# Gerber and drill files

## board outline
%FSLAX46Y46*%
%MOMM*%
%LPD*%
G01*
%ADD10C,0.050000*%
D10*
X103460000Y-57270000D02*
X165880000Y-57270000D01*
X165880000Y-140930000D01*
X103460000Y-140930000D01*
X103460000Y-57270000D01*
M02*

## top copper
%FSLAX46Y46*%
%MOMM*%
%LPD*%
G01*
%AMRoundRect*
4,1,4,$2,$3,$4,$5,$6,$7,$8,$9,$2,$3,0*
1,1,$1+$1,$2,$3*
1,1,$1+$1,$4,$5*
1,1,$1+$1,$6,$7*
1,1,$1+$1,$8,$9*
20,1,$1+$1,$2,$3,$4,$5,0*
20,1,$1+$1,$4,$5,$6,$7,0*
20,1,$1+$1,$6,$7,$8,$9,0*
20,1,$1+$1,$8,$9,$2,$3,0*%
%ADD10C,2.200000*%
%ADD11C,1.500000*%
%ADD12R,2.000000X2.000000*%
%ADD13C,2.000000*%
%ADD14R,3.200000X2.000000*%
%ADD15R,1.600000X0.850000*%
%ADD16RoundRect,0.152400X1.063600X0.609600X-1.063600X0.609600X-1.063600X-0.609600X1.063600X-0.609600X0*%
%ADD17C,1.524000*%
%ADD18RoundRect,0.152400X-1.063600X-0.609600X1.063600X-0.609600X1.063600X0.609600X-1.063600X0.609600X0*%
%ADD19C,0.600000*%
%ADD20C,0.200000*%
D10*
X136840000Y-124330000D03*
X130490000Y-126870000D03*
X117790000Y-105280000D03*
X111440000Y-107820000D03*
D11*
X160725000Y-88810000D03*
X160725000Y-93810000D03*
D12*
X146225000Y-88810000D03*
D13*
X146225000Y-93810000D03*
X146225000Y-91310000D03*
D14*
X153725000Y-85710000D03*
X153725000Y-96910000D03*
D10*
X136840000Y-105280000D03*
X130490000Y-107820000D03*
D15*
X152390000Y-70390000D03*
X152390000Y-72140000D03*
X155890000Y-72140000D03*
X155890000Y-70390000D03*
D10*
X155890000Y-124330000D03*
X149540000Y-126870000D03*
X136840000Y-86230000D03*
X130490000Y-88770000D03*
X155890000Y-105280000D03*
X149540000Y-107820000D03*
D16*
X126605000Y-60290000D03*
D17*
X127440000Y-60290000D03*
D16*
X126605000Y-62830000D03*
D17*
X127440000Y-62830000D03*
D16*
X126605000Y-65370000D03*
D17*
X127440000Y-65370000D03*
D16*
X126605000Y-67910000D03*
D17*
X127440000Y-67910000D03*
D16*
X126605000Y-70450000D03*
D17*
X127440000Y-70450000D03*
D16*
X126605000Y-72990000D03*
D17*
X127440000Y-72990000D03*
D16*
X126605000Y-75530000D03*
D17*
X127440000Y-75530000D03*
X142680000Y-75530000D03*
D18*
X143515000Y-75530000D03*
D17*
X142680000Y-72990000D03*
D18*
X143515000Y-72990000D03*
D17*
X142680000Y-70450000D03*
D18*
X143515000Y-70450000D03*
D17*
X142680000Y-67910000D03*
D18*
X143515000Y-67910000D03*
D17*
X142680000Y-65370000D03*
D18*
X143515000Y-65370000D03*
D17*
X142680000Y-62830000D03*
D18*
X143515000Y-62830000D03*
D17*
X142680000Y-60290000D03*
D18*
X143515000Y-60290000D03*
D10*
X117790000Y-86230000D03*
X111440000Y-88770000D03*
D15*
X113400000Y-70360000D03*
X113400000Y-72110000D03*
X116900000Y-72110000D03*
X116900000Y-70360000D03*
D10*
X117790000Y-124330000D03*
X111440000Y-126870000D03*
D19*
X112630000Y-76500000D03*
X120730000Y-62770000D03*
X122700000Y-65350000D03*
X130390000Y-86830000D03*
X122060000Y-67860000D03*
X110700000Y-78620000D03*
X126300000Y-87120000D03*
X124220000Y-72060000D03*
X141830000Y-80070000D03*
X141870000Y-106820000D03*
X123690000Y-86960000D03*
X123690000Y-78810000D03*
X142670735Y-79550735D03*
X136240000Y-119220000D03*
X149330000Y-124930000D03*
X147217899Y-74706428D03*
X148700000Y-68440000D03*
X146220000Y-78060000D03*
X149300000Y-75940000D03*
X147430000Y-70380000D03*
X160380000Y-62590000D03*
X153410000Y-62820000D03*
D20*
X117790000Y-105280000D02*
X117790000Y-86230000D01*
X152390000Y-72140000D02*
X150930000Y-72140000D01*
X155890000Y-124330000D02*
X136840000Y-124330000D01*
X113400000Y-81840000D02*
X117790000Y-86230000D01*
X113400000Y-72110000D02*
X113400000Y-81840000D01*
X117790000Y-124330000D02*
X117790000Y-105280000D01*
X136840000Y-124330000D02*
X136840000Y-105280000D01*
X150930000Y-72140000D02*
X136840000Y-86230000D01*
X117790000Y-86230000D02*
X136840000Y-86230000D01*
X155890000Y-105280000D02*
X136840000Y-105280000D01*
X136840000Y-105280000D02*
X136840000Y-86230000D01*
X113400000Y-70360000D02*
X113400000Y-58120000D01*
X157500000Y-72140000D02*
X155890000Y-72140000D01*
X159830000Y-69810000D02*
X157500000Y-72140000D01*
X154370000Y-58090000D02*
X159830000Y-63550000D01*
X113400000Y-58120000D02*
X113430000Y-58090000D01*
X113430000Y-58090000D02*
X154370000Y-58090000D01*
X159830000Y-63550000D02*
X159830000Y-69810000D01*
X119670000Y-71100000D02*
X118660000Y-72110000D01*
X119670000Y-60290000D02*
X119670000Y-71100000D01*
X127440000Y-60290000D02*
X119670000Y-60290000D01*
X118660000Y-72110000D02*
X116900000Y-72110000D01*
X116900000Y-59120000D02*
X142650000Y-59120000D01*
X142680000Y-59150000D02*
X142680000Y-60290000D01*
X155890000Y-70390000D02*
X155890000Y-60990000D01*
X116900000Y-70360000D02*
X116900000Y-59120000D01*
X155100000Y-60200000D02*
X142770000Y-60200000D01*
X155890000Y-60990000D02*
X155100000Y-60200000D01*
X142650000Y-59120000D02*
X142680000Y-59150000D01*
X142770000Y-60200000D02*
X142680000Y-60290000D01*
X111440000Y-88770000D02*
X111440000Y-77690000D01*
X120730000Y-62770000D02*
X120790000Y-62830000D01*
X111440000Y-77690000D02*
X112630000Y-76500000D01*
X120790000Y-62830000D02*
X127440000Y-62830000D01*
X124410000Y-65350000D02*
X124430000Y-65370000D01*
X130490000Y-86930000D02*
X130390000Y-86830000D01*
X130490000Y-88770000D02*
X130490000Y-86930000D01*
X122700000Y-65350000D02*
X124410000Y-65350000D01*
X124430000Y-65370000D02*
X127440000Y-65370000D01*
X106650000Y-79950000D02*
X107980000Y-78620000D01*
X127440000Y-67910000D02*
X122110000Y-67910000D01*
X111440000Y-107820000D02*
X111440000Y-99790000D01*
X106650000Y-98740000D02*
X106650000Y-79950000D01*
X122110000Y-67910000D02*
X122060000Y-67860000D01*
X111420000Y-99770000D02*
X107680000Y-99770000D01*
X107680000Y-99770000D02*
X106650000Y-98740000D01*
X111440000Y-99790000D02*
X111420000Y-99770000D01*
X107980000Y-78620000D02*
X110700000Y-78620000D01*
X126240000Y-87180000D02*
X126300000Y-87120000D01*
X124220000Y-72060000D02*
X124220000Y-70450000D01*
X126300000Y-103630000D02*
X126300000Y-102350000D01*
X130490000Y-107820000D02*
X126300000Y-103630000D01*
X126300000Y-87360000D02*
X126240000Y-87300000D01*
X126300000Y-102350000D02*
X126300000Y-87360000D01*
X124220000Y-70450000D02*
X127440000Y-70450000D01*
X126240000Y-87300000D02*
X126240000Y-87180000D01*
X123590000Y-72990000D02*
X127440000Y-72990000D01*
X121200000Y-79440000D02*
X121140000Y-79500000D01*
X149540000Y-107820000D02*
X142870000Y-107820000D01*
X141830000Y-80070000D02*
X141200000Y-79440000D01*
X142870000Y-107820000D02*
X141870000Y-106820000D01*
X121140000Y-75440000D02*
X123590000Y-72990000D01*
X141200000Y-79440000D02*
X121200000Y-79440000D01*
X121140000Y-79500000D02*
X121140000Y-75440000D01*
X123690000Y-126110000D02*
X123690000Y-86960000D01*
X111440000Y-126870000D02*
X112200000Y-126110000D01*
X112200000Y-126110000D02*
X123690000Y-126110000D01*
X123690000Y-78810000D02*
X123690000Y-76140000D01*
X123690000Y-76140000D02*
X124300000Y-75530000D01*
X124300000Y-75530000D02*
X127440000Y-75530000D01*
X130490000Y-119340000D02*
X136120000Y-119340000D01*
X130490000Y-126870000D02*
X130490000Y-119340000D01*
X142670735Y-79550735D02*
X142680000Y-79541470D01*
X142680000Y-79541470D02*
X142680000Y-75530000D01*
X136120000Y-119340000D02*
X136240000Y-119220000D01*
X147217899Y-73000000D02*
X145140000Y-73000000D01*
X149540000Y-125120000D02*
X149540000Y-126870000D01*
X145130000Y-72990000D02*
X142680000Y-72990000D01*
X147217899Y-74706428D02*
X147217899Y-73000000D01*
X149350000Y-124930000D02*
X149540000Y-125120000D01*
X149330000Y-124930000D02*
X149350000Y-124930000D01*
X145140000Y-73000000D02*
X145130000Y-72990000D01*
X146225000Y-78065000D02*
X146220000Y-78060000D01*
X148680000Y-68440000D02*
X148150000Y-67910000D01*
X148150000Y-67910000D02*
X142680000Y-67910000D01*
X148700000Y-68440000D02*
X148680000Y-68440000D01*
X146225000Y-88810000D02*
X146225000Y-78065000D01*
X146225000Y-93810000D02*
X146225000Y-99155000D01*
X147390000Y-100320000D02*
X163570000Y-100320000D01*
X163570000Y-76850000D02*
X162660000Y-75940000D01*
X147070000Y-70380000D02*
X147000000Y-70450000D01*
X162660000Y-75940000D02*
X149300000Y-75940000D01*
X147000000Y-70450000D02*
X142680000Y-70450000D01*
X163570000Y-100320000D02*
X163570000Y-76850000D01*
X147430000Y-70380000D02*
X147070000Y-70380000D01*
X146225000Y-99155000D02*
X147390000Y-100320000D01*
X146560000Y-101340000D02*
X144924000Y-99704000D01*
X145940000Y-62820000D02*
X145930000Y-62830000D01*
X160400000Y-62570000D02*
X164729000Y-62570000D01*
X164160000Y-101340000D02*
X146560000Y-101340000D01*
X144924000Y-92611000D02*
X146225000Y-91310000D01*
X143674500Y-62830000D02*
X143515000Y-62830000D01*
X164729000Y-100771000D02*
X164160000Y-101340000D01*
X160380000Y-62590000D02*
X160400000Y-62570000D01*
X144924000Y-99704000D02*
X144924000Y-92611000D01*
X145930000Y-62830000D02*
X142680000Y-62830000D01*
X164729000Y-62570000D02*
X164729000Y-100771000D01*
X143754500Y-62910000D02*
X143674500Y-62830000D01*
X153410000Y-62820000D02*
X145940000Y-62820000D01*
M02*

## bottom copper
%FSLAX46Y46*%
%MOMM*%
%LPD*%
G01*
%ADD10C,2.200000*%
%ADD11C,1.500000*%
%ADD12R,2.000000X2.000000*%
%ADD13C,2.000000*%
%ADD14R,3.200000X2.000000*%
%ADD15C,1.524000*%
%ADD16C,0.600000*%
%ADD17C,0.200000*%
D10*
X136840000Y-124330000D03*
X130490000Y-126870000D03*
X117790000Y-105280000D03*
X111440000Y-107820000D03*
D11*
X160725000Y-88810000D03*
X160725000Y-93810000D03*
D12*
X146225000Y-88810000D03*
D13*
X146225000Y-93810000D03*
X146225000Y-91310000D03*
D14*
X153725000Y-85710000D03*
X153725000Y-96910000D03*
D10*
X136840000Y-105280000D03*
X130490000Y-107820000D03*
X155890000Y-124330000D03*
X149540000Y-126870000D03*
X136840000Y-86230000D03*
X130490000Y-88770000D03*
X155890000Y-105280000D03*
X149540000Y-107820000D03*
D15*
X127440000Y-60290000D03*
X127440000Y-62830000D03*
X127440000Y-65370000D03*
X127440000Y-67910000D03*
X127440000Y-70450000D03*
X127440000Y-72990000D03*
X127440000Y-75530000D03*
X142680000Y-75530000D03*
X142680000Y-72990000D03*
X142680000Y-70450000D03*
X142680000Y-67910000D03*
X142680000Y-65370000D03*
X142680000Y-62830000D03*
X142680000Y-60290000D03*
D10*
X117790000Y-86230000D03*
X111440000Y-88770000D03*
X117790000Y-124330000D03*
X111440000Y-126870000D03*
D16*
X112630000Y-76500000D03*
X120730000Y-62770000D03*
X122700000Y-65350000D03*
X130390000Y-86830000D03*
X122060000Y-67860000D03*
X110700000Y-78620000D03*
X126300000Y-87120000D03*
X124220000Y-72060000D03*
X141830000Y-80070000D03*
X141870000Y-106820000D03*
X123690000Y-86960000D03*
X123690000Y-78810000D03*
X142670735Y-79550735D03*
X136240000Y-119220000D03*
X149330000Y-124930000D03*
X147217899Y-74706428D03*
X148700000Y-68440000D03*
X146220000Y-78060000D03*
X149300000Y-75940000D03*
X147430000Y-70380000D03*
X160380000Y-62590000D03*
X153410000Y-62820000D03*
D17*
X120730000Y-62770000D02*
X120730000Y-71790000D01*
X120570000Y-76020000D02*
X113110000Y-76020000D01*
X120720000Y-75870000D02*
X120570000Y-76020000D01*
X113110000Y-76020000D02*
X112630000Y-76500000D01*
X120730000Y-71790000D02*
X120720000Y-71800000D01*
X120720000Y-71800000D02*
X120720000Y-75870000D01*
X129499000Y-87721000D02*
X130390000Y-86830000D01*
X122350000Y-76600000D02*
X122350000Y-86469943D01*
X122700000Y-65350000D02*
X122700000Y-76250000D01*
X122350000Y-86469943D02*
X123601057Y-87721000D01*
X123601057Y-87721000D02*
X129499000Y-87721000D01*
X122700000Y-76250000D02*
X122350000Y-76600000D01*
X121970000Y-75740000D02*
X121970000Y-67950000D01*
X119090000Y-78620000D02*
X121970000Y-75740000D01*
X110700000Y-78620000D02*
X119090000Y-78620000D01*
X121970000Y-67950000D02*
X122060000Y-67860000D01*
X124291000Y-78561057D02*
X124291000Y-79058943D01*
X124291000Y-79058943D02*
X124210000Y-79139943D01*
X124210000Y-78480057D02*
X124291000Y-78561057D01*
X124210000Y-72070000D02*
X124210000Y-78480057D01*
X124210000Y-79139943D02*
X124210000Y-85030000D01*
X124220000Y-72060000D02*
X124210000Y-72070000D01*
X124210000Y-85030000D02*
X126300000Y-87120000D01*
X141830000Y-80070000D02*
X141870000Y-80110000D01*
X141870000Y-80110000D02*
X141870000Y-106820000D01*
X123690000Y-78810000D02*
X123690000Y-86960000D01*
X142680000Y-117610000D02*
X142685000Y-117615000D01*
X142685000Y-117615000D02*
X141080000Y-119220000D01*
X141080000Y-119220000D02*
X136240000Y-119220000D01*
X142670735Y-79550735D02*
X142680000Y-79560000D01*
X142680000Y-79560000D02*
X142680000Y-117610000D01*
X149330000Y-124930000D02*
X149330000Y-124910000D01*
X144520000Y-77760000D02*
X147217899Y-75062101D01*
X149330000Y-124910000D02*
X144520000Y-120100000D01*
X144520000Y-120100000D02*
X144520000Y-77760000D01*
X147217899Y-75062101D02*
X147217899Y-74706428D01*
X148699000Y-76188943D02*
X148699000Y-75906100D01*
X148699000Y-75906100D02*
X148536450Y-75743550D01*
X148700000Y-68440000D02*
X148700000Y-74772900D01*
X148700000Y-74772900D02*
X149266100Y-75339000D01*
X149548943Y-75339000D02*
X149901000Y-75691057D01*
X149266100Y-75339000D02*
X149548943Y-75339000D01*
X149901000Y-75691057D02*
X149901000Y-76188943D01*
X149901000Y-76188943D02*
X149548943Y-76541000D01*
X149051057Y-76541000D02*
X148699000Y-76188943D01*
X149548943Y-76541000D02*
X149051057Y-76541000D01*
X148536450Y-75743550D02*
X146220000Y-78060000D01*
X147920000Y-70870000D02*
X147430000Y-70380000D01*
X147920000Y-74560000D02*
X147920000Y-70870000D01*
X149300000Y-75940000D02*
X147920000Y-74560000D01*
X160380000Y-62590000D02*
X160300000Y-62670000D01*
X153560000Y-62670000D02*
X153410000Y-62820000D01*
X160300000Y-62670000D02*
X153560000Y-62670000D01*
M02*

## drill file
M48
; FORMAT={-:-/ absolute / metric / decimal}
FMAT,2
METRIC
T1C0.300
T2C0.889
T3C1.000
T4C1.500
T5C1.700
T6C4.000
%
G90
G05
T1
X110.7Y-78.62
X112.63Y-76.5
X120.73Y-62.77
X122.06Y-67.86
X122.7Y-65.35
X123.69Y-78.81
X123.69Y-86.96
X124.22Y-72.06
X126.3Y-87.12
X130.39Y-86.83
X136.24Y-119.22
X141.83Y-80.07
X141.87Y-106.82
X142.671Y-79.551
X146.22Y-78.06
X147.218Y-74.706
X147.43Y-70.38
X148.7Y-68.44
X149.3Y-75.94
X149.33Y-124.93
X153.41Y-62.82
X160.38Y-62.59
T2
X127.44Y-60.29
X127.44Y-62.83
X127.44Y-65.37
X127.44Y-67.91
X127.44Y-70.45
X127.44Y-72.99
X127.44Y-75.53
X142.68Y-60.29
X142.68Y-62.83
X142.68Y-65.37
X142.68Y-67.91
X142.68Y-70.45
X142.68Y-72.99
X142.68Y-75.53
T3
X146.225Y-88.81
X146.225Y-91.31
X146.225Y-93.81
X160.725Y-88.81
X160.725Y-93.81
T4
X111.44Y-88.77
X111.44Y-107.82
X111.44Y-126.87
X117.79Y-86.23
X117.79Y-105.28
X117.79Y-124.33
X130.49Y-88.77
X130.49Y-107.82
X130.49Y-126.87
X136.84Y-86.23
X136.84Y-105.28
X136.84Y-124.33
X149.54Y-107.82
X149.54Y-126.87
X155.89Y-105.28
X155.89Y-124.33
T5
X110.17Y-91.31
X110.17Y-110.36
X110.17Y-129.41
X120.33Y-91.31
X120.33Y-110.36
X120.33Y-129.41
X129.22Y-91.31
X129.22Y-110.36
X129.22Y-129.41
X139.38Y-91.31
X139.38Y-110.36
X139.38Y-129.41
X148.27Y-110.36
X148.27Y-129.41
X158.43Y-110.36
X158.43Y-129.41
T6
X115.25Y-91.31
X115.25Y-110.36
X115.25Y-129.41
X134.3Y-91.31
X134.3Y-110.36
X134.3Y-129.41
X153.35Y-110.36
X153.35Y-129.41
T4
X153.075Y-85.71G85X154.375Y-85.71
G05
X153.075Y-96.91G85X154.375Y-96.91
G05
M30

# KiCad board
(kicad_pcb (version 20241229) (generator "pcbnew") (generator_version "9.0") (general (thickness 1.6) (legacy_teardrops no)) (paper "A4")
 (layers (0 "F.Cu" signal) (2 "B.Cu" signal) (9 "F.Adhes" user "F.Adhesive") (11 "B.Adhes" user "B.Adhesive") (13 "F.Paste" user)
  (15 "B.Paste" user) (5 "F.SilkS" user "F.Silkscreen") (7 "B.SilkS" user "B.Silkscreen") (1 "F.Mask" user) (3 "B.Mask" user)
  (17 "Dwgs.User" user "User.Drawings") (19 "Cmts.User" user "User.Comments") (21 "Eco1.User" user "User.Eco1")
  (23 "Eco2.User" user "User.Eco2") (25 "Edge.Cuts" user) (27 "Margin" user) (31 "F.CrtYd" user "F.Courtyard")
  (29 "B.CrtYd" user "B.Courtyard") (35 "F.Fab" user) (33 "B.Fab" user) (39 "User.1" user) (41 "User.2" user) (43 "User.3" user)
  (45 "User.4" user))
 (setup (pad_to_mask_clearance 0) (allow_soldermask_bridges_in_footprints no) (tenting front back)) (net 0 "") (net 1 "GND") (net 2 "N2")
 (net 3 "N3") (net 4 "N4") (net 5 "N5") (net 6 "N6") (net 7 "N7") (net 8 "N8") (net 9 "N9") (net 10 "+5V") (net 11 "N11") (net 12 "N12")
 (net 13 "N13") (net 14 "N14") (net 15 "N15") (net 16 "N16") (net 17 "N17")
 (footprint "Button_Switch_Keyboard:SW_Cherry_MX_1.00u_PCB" (layer "F.Cu") (at 136.84 124.33)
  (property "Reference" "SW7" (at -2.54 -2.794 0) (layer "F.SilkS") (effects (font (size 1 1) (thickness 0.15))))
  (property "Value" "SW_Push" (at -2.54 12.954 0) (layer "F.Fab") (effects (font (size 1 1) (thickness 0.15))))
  (pad "" np_thru_hole circle (at -7.62 5.08) (size 1.7 1.7) (drill 1.7) (layers "*.Cu" "*.Mask"))
  (pad "" np_thru_hole circle (at -2.54 5.08) (size 4 4) (drill 4) (layers "*.Cu" "*.Mask"))
  (pad "" np_thru_hole circle (at 2.54 5.08) (size 1.7 1.7) (drill 1.7) (layers "*.Cu" "*.Mask"))
  (pad "1" thru_hole circle (at 0 0) (size 2.2 2.2) (drill 1.5) (layers "*.Cu" "*.Mask") (remove_unused_layers no) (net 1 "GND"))
  (pad "2" thru_hole circle (at -6.35 2.54) (size 2.2 2.2) (drill 1.5) (layers "*.Cu" "*.Mask") (remove_unused_layers no) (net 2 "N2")))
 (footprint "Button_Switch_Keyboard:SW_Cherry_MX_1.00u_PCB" (layer "F.Cu") (at 117.79 105.28)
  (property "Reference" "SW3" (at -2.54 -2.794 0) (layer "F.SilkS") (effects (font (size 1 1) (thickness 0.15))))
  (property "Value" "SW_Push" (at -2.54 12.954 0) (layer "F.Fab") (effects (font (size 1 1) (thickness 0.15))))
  (pad "" np_thru_hole circle (at -7.62 5.08) (size 1.7 1.7) (drill 1.7) (layers "*.Cu" "*.Mask"))
  (pad "" np_thru_hole circle (at -2.54 5.08) (size 4 4) (drill 4) (layers "*.Cu" "*.Mask"))
  (pad "" np_thru_hole circle (at 2.54 5.08) (size 1.7 1.7) (drill 1.7) (layers "*.Cu" "*.Mask"))
  (pad "1" thru_hole circle (at 0 0) (size 2.2 2.2) (drill 1.5) (layers "*.Cu" "*.Mask") (remove_unused_layers no) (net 1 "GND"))
  (pad "2" thru_hole circle (at -6.35 2.54) (size 2.2 2.2) (drill 1.5) (layers "*.Cu" "*.Mask") (remove_unused_layers no) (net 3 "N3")))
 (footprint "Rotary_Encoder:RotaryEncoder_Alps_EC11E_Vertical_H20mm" (layer "F.Cu") (at 146.225 88.81)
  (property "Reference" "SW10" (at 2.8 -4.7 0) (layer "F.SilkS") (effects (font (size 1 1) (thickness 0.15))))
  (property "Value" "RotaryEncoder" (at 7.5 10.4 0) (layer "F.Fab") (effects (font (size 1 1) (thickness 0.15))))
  (pad "" thru_hole circle (at 14.5 0) (size 1.5 1.5) (drill 1) (layers "*.Cu" "*.Mask") (remove_unused_layers no))
  (pad "" thru_hole circle (at 14.5 5) (size 1.5 1.5) (drill 1) (layers "*.Cu" "*.Mask") (remove_unused_layers no))
  (pad "A" thru_hole rect (at 0 0) (size 2 2) (drill 1) (layers "*.Cu" "*.Mask") (remove_unused_layers no) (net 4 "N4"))
  (pad "B" thru_hole circle (at 0 5) (size 2 2) (drill 1) (layers "*.Cu" "*.Mask") (remove_unused_layers no) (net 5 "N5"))
  (pad "C" thru_hole circle (at 0 2.5) (size 2 2) (drill 1) (layers "*.Cu" "*.Mask") (remove_unused_layers no) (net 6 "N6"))
  (pad "MP" thru_hole rect (at 7.5 -3.1) (size 3.2 2) (drill oval 2.8 1.5) (layers "*.Cu" "*.Mask") (remove_unused_layers no))
  (pad "MP" thru_hole rect (at 7.5 8.1) (size 3.2 2) (drill oval 2.8 1.5) (layers "*.Cu" "*.Mask") (remove_unused_layers no)))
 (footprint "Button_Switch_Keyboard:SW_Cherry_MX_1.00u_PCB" (layer "F.Cu") (at 136.84 105.28)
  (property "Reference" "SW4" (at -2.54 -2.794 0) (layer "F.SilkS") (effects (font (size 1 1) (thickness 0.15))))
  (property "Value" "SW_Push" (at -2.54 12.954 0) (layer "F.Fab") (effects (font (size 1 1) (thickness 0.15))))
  (pad "" np_thru_hole circle (at -7.62 5.08) (size 1.7 1.7) (drill 1.7) (layers "*.Cu" "*.Mask"))
  (pad "" np_thru_hole circle (at -2.54 5.08) (size 4 4) (drill 4) (layers "*.Cu" "*.Mask"))
  (pad "" np_thru_hole circle (at 2.54 5.08) (size 1.7 1.7) (drill 1.7) (layers "*.Cu" "*.Mask"))
  (pad "1" thru_hole circle (at 0 0) (size 2.2 2.2) (drill 1.5) (layers "*.Cu" "*.Mask") (remove_unused_layers no) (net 1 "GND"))
  (pad "2" thru_hole circle (at -6.35 2.54) (size 2.2 2.2) (drill 1.5) (layers "*.Cu" "*.Mask") (remove_unused_layers no) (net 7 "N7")))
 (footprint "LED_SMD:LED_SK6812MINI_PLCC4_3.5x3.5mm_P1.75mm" (layer "F.Cu") (at 154.14 71.265)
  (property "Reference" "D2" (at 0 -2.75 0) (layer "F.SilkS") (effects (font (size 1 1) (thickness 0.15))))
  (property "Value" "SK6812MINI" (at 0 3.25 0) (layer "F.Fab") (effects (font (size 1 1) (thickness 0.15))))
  (pad "1" smd rect (at -1.75 -0.875) (size 1.6 0.85) (layers "F.Cu" "F.Mask" "F.Paste") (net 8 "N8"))
  (pad "2" smd rect (at -1.75 0.875) (size 1.6 0.85) (layers "F.Cu" "F.Mask" "F.Paste") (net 1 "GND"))
  (pad "3" smd rect (at 1.75 0.875) (size 1.6 0.85) (layers "F.Cu" "F.Mask" "F.Paste") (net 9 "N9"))
  (pad "4" smd rect (at 1.75 -0.875) (size 1.6 0.85) (layers "F.Cu" "F.Mask" "F.Paste") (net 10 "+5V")))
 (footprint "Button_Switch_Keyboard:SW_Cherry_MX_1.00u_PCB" (layer "F.Cu") (at 155.89 124.33)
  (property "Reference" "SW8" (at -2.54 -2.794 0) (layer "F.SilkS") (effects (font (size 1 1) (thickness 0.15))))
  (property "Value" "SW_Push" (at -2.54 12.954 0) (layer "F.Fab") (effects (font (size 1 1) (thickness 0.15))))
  (pad "" np_thru_hole circle (at -7.62 5.08) (size 1.7 1.7) (drill 1.7) (layers "*.Cu" "*.Mask"))
  (pad "" np_thru_hole circle (at -2.54 5.08) (size 4 4) (drill 4) (layers "*.Cu" "*.Mask"))
  (pad "" np_thru_hole circle (at 2.54 5.08) (size 1.7 1.7) (drill 1.7) (layers "*.Cu" "*.Mask"))
  (pad "1" thru_hole circle (at 0 0) (size 2.2 2.2) (drill 1.5) (layers "*.Cu" "*.Mask") (remove_unused_layers no) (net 1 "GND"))
  (pad "2" thru_hole circle (at -6.35 2.54) (size 2.2 2.2) (drill 1.5) (layers "*.Cu" "*.Mask") (remove_unused_layers no) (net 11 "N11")))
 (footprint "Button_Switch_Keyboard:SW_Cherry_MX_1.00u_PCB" (layer "F.Cu") (at 136.84 86.23)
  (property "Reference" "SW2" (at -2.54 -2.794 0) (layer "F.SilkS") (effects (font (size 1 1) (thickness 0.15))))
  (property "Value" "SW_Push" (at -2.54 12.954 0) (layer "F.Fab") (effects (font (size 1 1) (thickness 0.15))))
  (pad "" np_thru_hole circle (at -7.62 5.08) (size 1.7 1.7) (drill 1.7) (layers "*.Cu" "*.Mask"))
  (pad "" np_thru_hole circle (at -2.54 5.08) (size 4 4) (drill 4) (layers "*.Cu" "*.Mask"))
  (pad "" np_thru_hole circle (at 2.54 5.08) (size 1.7 1.7) (drill 1.7) (layers "*.Cu" "*.Mask"))
  (pad "1" thru_hole circle (at 0 0) (size 2.2 2.2) (drill 1.5) (layers "*.Cu" "*.Mask") (remove_unused_layers no) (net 1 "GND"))
  (pad "2" thru_hole circle (at -6.35 2.54) (size 2.2 2.2) (drill 1.5) (layers "*.Cu" "*.Mask") (remove_unused_layers no) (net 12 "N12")))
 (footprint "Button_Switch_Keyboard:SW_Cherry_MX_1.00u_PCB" (layer "F.Cu") (at 155.89 105.28)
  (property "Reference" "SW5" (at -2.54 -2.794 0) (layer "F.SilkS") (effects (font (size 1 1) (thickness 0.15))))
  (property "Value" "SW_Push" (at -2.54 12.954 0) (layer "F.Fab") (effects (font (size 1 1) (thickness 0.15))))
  (pad "" np_thru_hole circle (at -7.62 5.08) (size 1.7 1.7) (drill 1.7) (layers "*.Cu" "*.Mask"))
  (pad "" np_thru_hole circle (at -2.54 5.08) (size 4 4) (drill 4) (layers "*.Cu" "*.Mask"))
  (pad "" np_thru_hole circle (at 2.54 5.08) (size 1.7 1.7) (drill 1.7) (layers "*.Cu" "*.Mask"))
  (pad "1" thru_hole circle (at 0 0) (size 2.2 2.2) (drill 1.5) (layers "*.Cu" "*.Mask") (remove_unused_layers no) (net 1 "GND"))
  (pad "2" thru_hole circle (at -6.35 2.54) (size 2.2 2.2) (drill 1.5) (layers "*.Cu" "*.Mask") (remove_unused_layers no) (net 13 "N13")))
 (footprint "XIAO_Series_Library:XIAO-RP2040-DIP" (layer "F.Cu") (at 135.06 67.91)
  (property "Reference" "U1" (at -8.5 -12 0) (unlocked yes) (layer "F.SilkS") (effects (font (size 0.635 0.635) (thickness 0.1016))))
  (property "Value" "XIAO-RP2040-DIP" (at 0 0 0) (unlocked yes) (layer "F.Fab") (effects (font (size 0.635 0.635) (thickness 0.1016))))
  (pad "1" smd roundrect (at -8.455 -7.62 180) (size 2.432 1.524) (layers "F.Cu" "F.Mask") (roundrect_rratio 0.1) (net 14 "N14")
   (thermal_bridge_angle 45))
  (pad "1" thru_hole circle (at -7.62 -7.62 180) (size 1.524 1.524) (drill 0.889) (layers "*.Cu" "*.Mask") (remove_unused_layers no)
   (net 14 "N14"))
  (pad "2" smd roundrect (at -8.455 -5.08 180) (size 2.432 1.524) (layers "F.Cu" "F.Mask") (roundrect_rratio 0.1) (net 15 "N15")
   (thermal_bridge_angle 45))
  (pad "2" thru_hole circle (at -7.62 -5.08 180) (size 1.524 1.524) (drill 0.889) (layers "*.Cu" "*.Mask") (remove_unused_layers no)
   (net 15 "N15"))
  (pad "3" smd roundrect (at -8.455 -2.54 180) (size 2.432 1.524) (layers "F.Cu" "F.Mask") (roundrect_rratio 0.1) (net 12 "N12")
   (thermal_bridge_angle 45))
  (pad "3" thru_hole circle (at -7.62 -2.54 180) (size 1.524 1.524) (drill 0.889) (layers "*.Cu" "*.Mask") (remove_unused_layers no)
   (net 12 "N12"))
  (pad "4" smd roundrect (at -8.455 0 180) (size 2.432 1.524) (layers "F.Cu" "F.Mask") (roundrect_rratio 0.1) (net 3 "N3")
   (thermal_bridge_angle 45))
  (pad "4" thru_hole circle (at -7.62 0 180) (size 1.524 1.524) (drill 0.889) (layers "*.Cu" "*.Mask") (remove_unused_layers no)
   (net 3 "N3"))
  (pad "5" smd roundrect (at -8.455 2.54 180) (size 2.432 1.524) (layers "F.Cu" "F.Mask") (roundrect_rratio 0.1) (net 7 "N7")
   (thermal_bridge_angle 45))
  (pad "5" thru_hole circle (at -7.62 2.54 180) (size 1.524 1.524) (drill 0.889) (layers "*.Cu" "*.Mask") (remove_unused_layers no)
   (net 7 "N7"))
  (pad "6" smd roundrect (at -8.455 5.08 180) (size 2.432 1.524) (layers "F.Cu" "F.Mask") (roundrect_rratio 0.1) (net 13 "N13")
   (thermal_bridge_angle 45))
  (pad "6" thru_hole circle (at -7.62 5.08 180) (size 1.524 1.524) (drill 0.889) (layers "*.Cu" "*.Mask") (remove_unused_layers no)
   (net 13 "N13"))
  (pad "7" smd roundrect (at -8.455 7.62 180) (size 2.432 1.524) (layers "F.Cu" "F.Mask") (roundrect_rratio 0.1) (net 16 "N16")
   (thermal_bridge_angle 45))
  (pad "7" thru_hole circle (at -7.62 7.62 180) (size 1.524 1.524) (drill 0.889) (layers "*.Cu" "*.Mask") (remove_unused_layers no)
   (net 16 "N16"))
  (pad "8" thru_hole circle (at 7.62 7.62) (size 1.524 1.524) (drill 0.889) (layers "*.Cu" "*.Mask") (remove_unused_layers no) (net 2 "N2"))
  (pad "8" smd roundrect (at 8.455 7.62) (size 2.432 1.524) (layers "F.Cu" "F.Mask") (roundrect_rratio 0.1) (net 2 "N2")
   (thermal_bridge_angle 45))
  (pad "9" thru_hole circle (at 7.62 5.08) (size 1.524 1.524) (drill 0.889) (layers "*.Cu" "*.Mask") (remove_unused_layers no)
   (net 11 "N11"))
  (pad "9" smd roundrect (at 8.455 5.08) (size 2.432 1.524) (layers "F.Cu" "F.Mask") (roundrect_rratio 0.1) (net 11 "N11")
   (thermal_bridge_angle 45))
  (pad "10" thru_hole circle (at 7.62 2.54) (size 1.524 1.524) (drill 0.889) (layers "*.Cu" "*.Mask") (remove_unused_layers no) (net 5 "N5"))
  (pad "10" smd roundrect (at 8.455 2.54) (size 2.432 1.524) (layers "F.Cu" "F.Mask") (roundrect_rratio 0.1) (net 5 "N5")
   (thermal_bridge_angle 45))
  (pad "11" thru_hole circle (at 7.62 0) (size 1.524 1.524) (drill 0.889) (layers "*.Cu" "*.Mask") (remove_unused_layers no) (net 4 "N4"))
  (pad "11" smd roundrect (at 8.455 0) (size 2.432 1.524) (layers "F.Cu" "F.Mask") (roundrect_rratio 0.1) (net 4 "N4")
   (thermal_bridge_angle 45))
  (pad "12" thru_hole circle (at 7.62 -2.54) (size 1.524 1.524) (drill 0.889) (layers "*.Cu" "*.Mask") (remove_unused_layers no)
   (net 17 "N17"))
  (pad "12" smd roundrect (at 8.455 -2.54) (size 2.432 1.524) (layers "F.Cu" "F.Mask") (roundrect_rratio 0.1) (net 17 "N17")
   (thermal_bridge_angle 45))
  (pad "13" thru_hole circle (at 7.62 -5.08) (size 1.524 1.524) (drill 0.889) (layers "*.Cu" "*.Mask") (remove_unused_layers no)
   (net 6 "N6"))
  (pad "13" smd roundrect (at 8.455 -5.08) (size 2.432 1.524) (layers "F.Cu" "F.Mask") (roundrect_rratio 0.1) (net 6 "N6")
   (thermal_bridge_angle 45))
  (pad "14" thru_hole circle (at 7.62 -7.62) (size 1.524 1.524) (drill 0.889) (layers "*.Cu" "*.Mask") (remove_unused_layers no)
   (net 10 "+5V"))
  (pad "14" smd roundrect (at 8.455 -7.62) (size 2.432 1.524) (layers "F.Cu" "F.Mask") (roundrect_rratio 0.1) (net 10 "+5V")
   (thermal_bridge_angle 45)))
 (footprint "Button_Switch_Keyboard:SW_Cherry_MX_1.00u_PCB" (layer "F.Cu") (at 117.79 86.23)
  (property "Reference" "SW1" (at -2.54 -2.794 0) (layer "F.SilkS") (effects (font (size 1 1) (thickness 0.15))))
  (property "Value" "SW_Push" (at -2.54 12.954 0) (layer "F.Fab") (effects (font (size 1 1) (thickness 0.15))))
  (pad "" np_thru_hole circle (at -7.62 5.08) (size 1.7 1.7) (drill 1.7) (layers "*.Cu" "*.Mask"))
  (pad "" np_thru_hole circle (at -2.54 5.08) (size 4 4) (drill 4) (layers "*.Cu" "*.Mask"))
  (pad "" np_thru_hole circle (at 2.54 5.08) (size 1.7 1.7) (drill 1.7) (layers "*.Cu" "*.Mask"))
  (pad "1" thru_hole circle (at 0 0) (size 2.2 2.2) (drill 1.5) (layers "*.Cu" "*.Mask") (remove_unused_layers no) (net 1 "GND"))
  (pad "2" thru_hole circle (at -6.35 2.54) (size 2.2 2.2) (drill 1.5) (layers "*.Cu" "*.Mask") (remove_unused_layers no) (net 15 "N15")))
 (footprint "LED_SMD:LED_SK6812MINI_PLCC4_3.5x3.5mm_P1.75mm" (layer "F.Cu") (at 115.15 71.235)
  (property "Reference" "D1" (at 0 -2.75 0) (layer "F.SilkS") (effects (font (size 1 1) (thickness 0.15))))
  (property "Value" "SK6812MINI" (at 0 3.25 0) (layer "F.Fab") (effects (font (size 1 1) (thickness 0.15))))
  (pad "1" smd rect (at -1.75 -0.875) (size 1.6 0.85) (layers "F.Cu" "F.Mask" "F.Paste") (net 9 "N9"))
  (pad "2" smd rect (at -1.75 0.875) (size 1.6 0.85) (layers "F.Cu" "F.Mask" "F.Paste") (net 1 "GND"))
  (pad "3" smd rect (at 1.75 0.875) (size 1.6 0.85) (layers "F.Cu" "F.Mask" "F.Paste") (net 14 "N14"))
  (pad "4" smd rect (at 1.75 -0.875) (size 1.6 0.85) (layers "F.Cu" "F.Mask" "F.Paste") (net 10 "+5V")))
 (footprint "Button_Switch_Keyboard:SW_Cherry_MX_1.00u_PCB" (layer "F.Cu") (at 117.79 124.33)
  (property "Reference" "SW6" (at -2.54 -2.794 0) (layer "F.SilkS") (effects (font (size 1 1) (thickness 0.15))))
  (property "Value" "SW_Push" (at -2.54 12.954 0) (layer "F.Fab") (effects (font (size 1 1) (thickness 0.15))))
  (pad "" np_thru_hole circle (at -7.62 5.08) (size 1.7 1.7) (drill 1.7) (layers "*.Cu" "*.Mask"))
  (pad "" np_thru_hole circle (at -2.54 5.08) (size 4 4) (drill 4) (layers "*.Cu" "*.Mask"))
  (pad "" np_thru_hole circle (at 2.54 5.08) (size 1.7 1.7) (drill 1.7) (layers "*.Cu" "*.Mask"))
  (pad "1" thru_hole circle (at 0 0) (size 2.2 2.2) (drill 1.5) (layers "*.Cu" "*.Mask") (remove_unused_layers no) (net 1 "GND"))
  (pad "2" thru_hole circle (at -6.35 2.54) (size 2.2 2.2) (drill 1.5) (layers "*.Cu" "*.Mask") (remove_unused_layers no) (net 16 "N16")))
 (gr_rect (start 103.46 57.27) (end 165.88 140.93) (stroke (width 0.05) (type default)) (fill no) (layer "Edge.Cuts"))
 (segment (start 117.79 105.28) (end 117.79 86.23) (width 0.2) (layer "F.Cu") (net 1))
 (segment (start 152.39 72.14) (end 150.93 72.14) (width 0.2) (layer "F.Cu") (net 1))
 (segment (start 155.89 124.33) (end 136.84 124.33) (width 0.2) (layer "F.Cu") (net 1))
 (segment (start 113.4 81.84) (end 117.79 86.23) (width 0.2) (layer "F.Cu") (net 1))
 (segment (start 113.4 72.11) (end 113.4 81.84) (width 0.2) (layer "F.Cu") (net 1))
 (segment (start 117.79 124.33) (end 117.79 105.28) (width 0.2) (layer "F.Cu") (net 1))
 (segment (start 136.84 124.33) (end 136.84 105.28) (width 0.2) (layer "F.Cu") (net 1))
 (segment (start 150.93 72.14) (end 136.84 86.23) (width 0.2) (layer "F.Cu") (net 1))
 (segment (start 117.79 86.23) (end 136.84 86.23) (width 0.2) (layer "F.Cu") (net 1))
 (segment (start 155.89 105.28) (end 136.84 105.28) (width 0.2) (layer "F.Cu") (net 1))
 (segment (start 136.84 105.28) (end 136.84 86.23) (width 0.2) (layer "F.Cu") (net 1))
 (segment (start 113.4 70.36) (end 113.4 58.12) (width 0.2) (layer "F.Cu") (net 9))
 (segment (start 157.5 72.14) (end 155.89 72.14) (width 0.2) (layer "F.Cu") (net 9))
 (segment (start 159.83 69.81) (end 157.5 72.14) (width 0.2) (layer "F.Cu") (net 9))
 (segment (start 154.37 58.09) (end 159.83 63.55) (width 0.2) (layer "F.Cu") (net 9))
 (segment (start 113.4 58.12) (end 113.43 58.09) (width 0.2) (layer "F.Cu") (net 9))
 (segment (start 113.43 58.09) (end 154.37 58.09) (width 0.2) (layer "F.Cu") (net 9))
 (segment (start 159.83 63.55) (end 159.83 69.81) (width 0.2) (layer "F.Cu") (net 9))
 (segment (start 119.67 71.1) (end 118.66 72.11) (width 0.2) (layer "F.Cu") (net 14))
 (segment (start 119.67 60.29) (end 119.67 71.1) (width 0.2) (layer "F.Cu") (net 14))
 (segment (start 127.44 60.29) (end 119.67 60.29) (width 0.2) (layer "F.Cu") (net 14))
 (segment (start 118.66 72.11) (end 116.9 72.11) (width 0.2) (layer "F.Cu") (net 14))
 (segment (start 116.9 59.12) (end 142.65 59.12) (width 0.2) (layer "F.Cu") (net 10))
 (segment (start 142.68 59.15) (end 142.68 60.29) (width 0.2) (layer "F.Cu") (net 10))
 (segment (start 155.89 70.39) (end 155.89 60.99) (width 0.2) (layer "F.Cu") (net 10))
 (segment (start 116.9 70.36) (end 116.9 59.12) (width 0.2) (layer "F.Cu") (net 10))
 (segment (start 155.1 60.2) (end 142.77 60.2) (width 0.2) (layer "F.Cu") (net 10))
 (segment (start 155.89 60.99) (end 155.1 60.2) (width 0.2) (layer "F.Cu") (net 10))
 (segment (start 142.65 59.12) (end 142.68 59.15) (width 0.2) (layer "F.Cu") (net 10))
 (segment (start 142.77 60.2) (end 142.68 60.29) (width 0.2) (layer "F.Cu") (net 10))
 (segment (start 111.44 88.77) (end 111.44 77.69) (width 0.2) (layer "F.Cu") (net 15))
 (segment (start 120.73 62.77) (end 120.79 62.83) (width 0.2) (layer "F.Cu") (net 15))
 (segment (start 111.44 77.69) (end 112.63 76.5) (width 0.2) (layer "F.Cu") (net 15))
 (segment (start 120.79 62.83) (end 127.44 62.83) (width 0.2) (layer "F.Cu") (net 15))
 (via (at 112.63 76.5) (size 0.6) (drill 0.3) (layers "F.Cu" "B.Cu") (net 15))
 (via (at 120.73 62.77) (size 0.6) (drill 0.3) (layers "F.Cu" "B.Cu") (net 15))
 (segment (start 120.73 62.77) (end 120.73 71.79) (width 0.2) (layer "B.Cu") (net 15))
 (segment (start 120.57 76.02) (end 113.11 76.02) (width 0.2) (layer "B.Cu") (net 15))
 (segment (start 120.72 75.87) (end 120.57 76.02) (width 0.2) (layer "B.Cu") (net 15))
 (segment (start 113.11 76.02) (end 112.63 76.5) (width 0.2) (layer "B.Cu") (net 15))
 (segment (start 120.73 71.79) (end 120.72 71.8) (width 0.2) (layer "B.Cu") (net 15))
 (segment (start 120.72 71.8) (end 120.72 75.87) (width 0.2) (layer "B.Cu") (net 15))
 (segment (start 124.41 65.35) (end 124.43 65.37) (width 0.2) (layer "F.Cu") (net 12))
 (segment (start 130.49 86.93) (end 130.39 86.83) (width 0.2) (layer "F.Cu") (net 12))
 (segment (start 130.49 88.77) (end 130.49 86.93) (width 0.2) (layer "F.Cu") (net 12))
 (segment (start 122.7 65.35) (end 124.41 65.35) (width 0.2) (layer "F.Cu") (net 12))
 (segment (start 124.43 65.37) (end 127.44 65.37) (width 0.2) (layer "F.Cu") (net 12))
 (via (at 122.7 65.35) (size 0.6) (drill 0.3) (layers "F.Cu" "B.Cu") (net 12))
 (via (at 130.39 86.83) (size 0.6) (drill 0.3) (layers "F.Cu" "B.Cu") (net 12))
 (segment (start 129.499 87.721) (end 130.39 86.83) (width 0.2) (layer "B.Cu") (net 12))
 (segment (start 122.35 76.6) (end 122.35 86.469943) (width 0.2) (layer "B.Cu") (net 12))
 (segment (start 122.7 65.35) (end 122.7 76.25) (width 0.2) (layer "B.Cu") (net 12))
 (segment (start 122.35 86.469943) (end 123.601057 87.721) (width 0.2) (layer "B.Cu") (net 12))
 (segment (start 123.601057 87.721) (end 129.499 87.721) (width 0.2) (layer "B.Cu") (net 12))
 (segment (start 122.7 76.25) (end 122.35 76.6) (width 0.2) (layer "B.Cu") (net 12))
 (segment (start 106.65 79.95) (end 107.98 78.62) (width 0.2) (layer "F.Cu") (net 3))
 (segment (start 127.44 67.91) (end 122.11 67.91) (width 0.2) (layer "F.Cu") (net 3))
 (segment (start 111.44 107.82) (end 111.44 99.79) (width 0.2) (layer "F.Cu") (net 3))
 (segment (start 106.65 98.74) (end 106.65 79.95) (width 0.2) (layer "F.Cu") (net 3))
 (segment (start 122.11 67.91) (end 122.06 67.86) (width 0.2) (layer "F.Cu") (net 3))
 (segment (start 111.42 99.77) (end 107.68 99.77) (width 0.2) (layer "F.Cu") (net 3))
 (segment (start 107.68 99.77) (end 106.65 98.74) (width 0.2) (layer "F.Cu") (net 3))
 (segment (start 111.44 99.79) (end 111.42 99.77) (width 0.2) (layer "F.Cu") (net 3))
 (segment (start 107.98 78.62) (end 110.7 78.62) (width 0.2) (layer "F.Cu") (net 3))
 (via (at 122.06 67.86) (size 0.6) (drill 0.3) (layers "F.Cu" "B.Cu") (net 3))
 (via (at 110.7 78.62) (size 0.6) (drill 0.3) (layers "F.Cu" "B.Cu") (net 3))
 (segment (start 121.97 75.74) (end 121.97 67.95) (width 0.2) (layer "B.Cu") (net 3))
 (segment (start 119.09 78.62) (end 121.97 75.74) (width 0.2) (layer "B.Cu") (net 3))
 (segment (start 110.7 78.62) (end 119.09 78.62) (width 0.2) (layer "B.Cu") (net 3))
 (segment (start 121.97 67.95) (end 122.06 67.86) (width 0.2) (layer "B.Cu") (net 3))
 (segment (start 126.24 87.18) (end 126.3 87.12) (width 0.2) (layer "F.Cu") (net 7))
 (segment (start 124.22 72.06) (end 124.22 70.45) (width 0.2) (layer "F.Cu") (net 7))
 (segment (start 126.3 103.63) (end 126.3 102.35) (width 0.2) (layer "F.Cu") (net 7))
 (segment (start 130.49 107.82) (end 126.3 103.63) (width 0.2) (layer "F.Cu") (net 7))
 (segment (start 126.3 87.36) (end 126.24 87.3) (width 0.2) (layer "F.Cu") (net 7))
 (segment (start 126.3 102.35) (end 126.3 87.36) (width 0.2) (layer "F.Cu") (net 7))
 (segment (start 124.22 70.45) (end 127.44 70.45) (width 0.2) (layer "F.Cu") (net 7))
 (segment (start 126.24 87.3) (end 126.24 87.18) (width 0.2) (layer "F.Cu") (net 7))
 (via (at 126.3 87.12) (size 0.6) (drill 0.3) (layers "F.Cu" "B.Cu") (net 7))
 (via (at 124.22 72.06) (size 0.6) (drill 0.3) (layers "F.Cu" "B.Cu") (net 7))
 (segment (start 124.291 78.561057) (end 124.291 79.058943) (width 0.2) (layer "B.Cu") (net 7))
 (segment (start 124.291 79.058943) (end 124.21 79.139943) (width 0.2) (layer "B.Cu") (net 7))
 (segment (start 124.21 78.480057) (end 124.291 78.561057) (width 0.2) (layer "B.Cu") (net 7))
 (segment (start 124.21 72.07) (end 124.21 78.480057) (width 0.2) (layer "B.Cu") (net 7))
 (segment (start 124.21 79.139943) (end 124.21 85.03) (width 0.2) (layer "B.Cu") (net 7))
 (segment (start 124.22 72.06) (end 124.21 72.07) (width 0.2) (layer "B.Cu") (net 7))
 (segment (start 124.21 85.03) (end 126.3 87.12) (width 0.2) (layer "B.Cu") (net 7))
 (segment (start 123.59 72.99) (end 127.44 72.99) (width 0.2) (layer "F.Cu") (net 13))
 (segment (start 121.2 79.44) (end 121.14 79.5) (width 0.2) (layer "F.Cu") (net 13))
 (segment (start 149.54 107.82) (end 142.87 107.82) (width 0.2) (layer "F.Cu") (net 13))
 (segment (start 141.83 80.07) (end 141.2 79.44) (width 0.2) (layer "F.Cu") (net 13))
 (segment (start 142.87 107.82) (end 141.87 106.82) (width 0.2) (layer "F.Cu") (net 13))
 (segment (start 121.14 75.44) (end 123.59 72.99) (width 0.2) (layer "F.Cu") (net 13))
 (segment (start 141.2 79.44) (end 121.2 79.44) (width 0.2) (layer "F.Cu") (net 13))
 (segment (start 121.14 79.5) (end 121.14 75.44) (width 0.2) (layer "F.Cu") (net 13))
 (via (at 141.83 80.07) (size 0.6) (drill 0.3) (layers "F.Cu" "B.Cu") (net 13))
 (via (at 141.87 106.82) (size 0.6) (drill 0.3) (layers "F.Cu" "B.Cu") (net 13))
 (segment (start 141.83 80.07) (end 141.87 80.11) (width 0.2) (layer "B.Cu") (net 13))
 (segment (start 141.87 80.11) (end 141.87 106.82) (width 0.2) (layer "B.Cu") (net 13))
 (segment (start 123.69 126.11) (end 123.69 86.96) (width 0.2) (layer "F.Cu") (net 16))
 (segment (start 111.44 126.87) (end 112.2 126.11) (width 0.2) (layer "F.Cu") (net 16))
 (segment (start 112.2 126.11) (end 123.69 126.11) (width 0.2) (layer "F.Cu") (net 16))
 (segment (start 123.69 78.81) (end 123.69 76.14) (width 0.2) (layer "F.Cu") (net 16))
 (segment (start 123.69 76.14) (end 124.3 75.53) (width 0.2) (layer "F.Cu") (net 16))
 (segment (start 124.3 75.53) (end 127.44 75.53) (width 0.2) (layer "F.Cu") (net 16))
 (via (at 123.69 86.96) (size 0.6) (drill 0.3) (layers "F.Cu" "B.Cu") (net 16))
 (via (at 123.69 78.81) (size 0.6) (drill 0.3) (layers "F.Cu" "B.Cu") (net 16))
 (segment (start 123.69 78.81) (end 123.69 86.96) (width 0.2) (layer "B.Cu") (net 16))
 (segment (start 130.49 119.34) (end 136.12 119.34) (width 0.2) (layer "F.Cu") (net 2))
 (segment (start 130.49 126.87) (end 130.49 119.34) (width 0.2) (layer "F.Cu") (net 2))
 (segment (start 142.670735 79.550735) (end 142.68 79.54147) (width 0.2) (layer "F.Cu") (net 2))
 (segment (start 142.68 79.54147) (end 142.68 75.53) (width 0.2) (layer "F.Cu") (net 2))
 (segment (start 136.12 119.34) (end 136.24 119.22) (width 0.2) (layer "F.Cu") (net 2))
 (via (at 142.670735 79.550735) (size 0.6) (drill 0.3) (layers "F.Cu" "B.Cu") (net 2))
 (via (at 136.24 119.22) (size 0.6) (drill 0.3) (layers "F.Cu" "B.Cu") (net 2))
 (segment (start 142.68 117.61) (end 142.685 117.615) (width 0.2) (layer "B.Cu") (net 2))
 (segment (start 142.685 117.615) (end 141.08 119.22) (width 0.2) (layer "B.Cu") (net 2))
 (segment (start 141.08 119.22) (end 136.24 119.22) (width 0.2) (layer "B.Cu") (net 2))
 (segment (start 142.670735 79.550735) (end 142.68 79.56) (width 0.2) (layer "B.Cu") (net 2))
 (segment (start 142.68 79.56) (end 142.68 117.61) (width 0.2) (layer "B.Cu") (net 2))
 (segment (start 147.217899 73) (end 145.14 73) (width 0.2) (layer "F.Cu") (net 11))
 (segment (start 149.54 125.12) (end 149.54 126.87) (width 0.2) (layer "F.Cu") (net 11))
 (segment (start 145.13 72.99) (end 142.68 72.99) (width 0.2) (layer "F.Cu") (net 11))
 (segment (start 147.217899 74.706428) (end 147.217899 73) (width 0.2) (layer "F.Cu") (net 11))
 (segment (start 149.35 124.93) (end 149.54 125.12) (width 0.2) (layer "F.Cu") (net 11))
 (segment (start 149.33 124.93) (end 149.35 124.93) (width 0.2) (layer "F.Cu") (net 11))
 (segment (start 145.14 73) (end 145.13 72.99) (width 0.2) (layer "F.Cu") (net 11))
 (via (at 149.33 124.93) (size 0.6) (drill 0.3) (layers "F.Cu" "B.Cu") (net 11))
 (via (at 147.217899 74.706428) (size 0.6) (drill 0.3) (layers "F.Cu" "B.Cu") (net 11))
 (segment (start 149.33 124.93) (end 149.33 124.91) (width 0.2) (layer "B.Cu") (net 11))
 (segment (start 144.52 77.76) (end 147.217899 75.062101) (width 0.2) (layer "B.Cu") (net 11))
 (segment (start 149.33 124.91) (end 144.52 120.1) (width 0.2) (layer "B.Cu") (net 11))
 (segment (start 144.52 120.1) (end 144.52 77.76) (width 0.2) (layer "B.Cu") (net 11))
 (segment (start 147.217899 75.062101) (end 147.217899 74.706428) (width 0.2) (layer "B.Cu") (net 11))
 (segment (start 146.225 78.065) (end 146.22 78.06) (width 0.2) (layer "F.Cu") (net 4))
 (segment (start 148.68 68.44) (end 148.15 67.91) (width 0.2) (layer "F.Cu") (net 4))
 (segment (start 148.15 67.91) (end 142.68 67.91) (width 0.2) (layer "F.Cu") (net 4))
 (segment (start 148.7 68.44) (end 148.68 68.44) (width 0.2) (layer "F.Cu") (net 4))
 (segment (start 146.225 88.81) (end 146.225 78.065) (width 0.2) (layer "F.Cu") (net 4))
 (via (at 148.7 68.44) (size 0.6) (drill 0.3) (layers "F.Cu" "B.Cu") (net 4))
 (via (at 146.22 78.06) (size 0.6) (drill 0.3) (layers "F.Cu" "B.Cu") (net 4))
 (segment (start 148.699 76.188943) (end 148.699 75.9061) (width 0.2) (layer "B.Cu") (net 4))
 (segment (start 148.699 75.9061) (end 148.53645 75.74355) (width 0.2) (layer "B.Cu") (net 4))
 (segment (start 148.7 68.44) (end 148.7 74.7729) (width 0.2) (layer "B.Cu") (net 4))
 (segment (start 148.7 74.7729) (end 149.2661 75.339) (width 0.2) (layer "B.Cu") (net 4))
 (segment (start 149.548943 75.339) (end 149.901 75.691057) (width 0.2) (layer "B.Cu") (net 4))
 (segment (start 149.2661 75.339) (end 149.548943 75.339) (width 0.2) (layer "B.Cu") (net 4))
 (segment (start 149.901 75.691057) (end 149.901 76.188943) (width 0.2) (layer "B.Cu") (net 4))
 (segment (start 149.901 76.188943) (end 149.548943 76.541) (width 0.2) (layer "B.Cu") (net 4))
 (segment (start 149.051057 76.541) (end 148.699 76.188943) (width 0.2) (layer "B.Cu") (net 4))
 (segment (start 149.548943 76.541) (end 149.051057 76.541) (width 0.2) (layer "B.Cu") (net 4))
 (segment (start 148.53645 75.74355) (end 146.22 78.06) (width 0.2) (layer "B.Cu") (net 4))
 (segment (start 146.225 93.81) (end 146.225 99.155) (width 0.2) (layer "F.Cu") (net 5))
 (segment (start 147.39 100.32) (end 163.57 100.32) (width 0.2) (layer "F.Cu") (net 5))
 (segment (start 163.57 76.85) (end 162.66 75.94) (width 0.2) (layer "F.Cu") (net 5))
 (segment (start 147.07 70.38) (end 147 70.45) (width 0.2) (layer "F.Cu") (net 5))
 (segment (start 162.66 75.94) (end 149.3 75.94) (width 0.2) (layer "F.Cu") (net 5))
 (segment (start 147 70.45) (end 142.68 70.45) (width 0.2) (layer "F.Cu") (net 5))
 (segment (start 163.57 100.32) (end 163.57 76.85) (width 0.2) (layer "F.Cu") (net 5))
 (segment (start 147.43 70.38) (end 147.07 70.38) (width 0.2) (layer "F.Cu") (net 5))
 (segment (start 146.225 99.155) (end 147.39 100.32) (width 0.2) (layer "F.Cu") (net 5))
 (via (at 149.3 75.94) (size 0.6) (drill 0.3) (layers "F.Cu" "B.Cu") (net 5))
 (via (at 147.43 70.38) (size 0.6) (drill 0.3) (layers "F.Cu" "B.Cu") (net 5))
 (segment (start 147.92 70.87) (end 147.43 70.38) (width 0.2) (layer "B.Cu") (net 5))
 (segment (start 147.92 74.56) (end 147.92 70.87) (width 0.2) (layer "B.Cu") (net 5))
 (segment (start 149.3 75.94) (end 147.92 74.56) (width 0.2) (layer "B.Cu") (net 5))
 (segment (start 146.56 101.34) (end 144.924 99.704) (width 0.2) (layer "F.Cu") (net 6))
 (segment (start 145.94 62.82) (end 145.93 62.83) (width 0.2) (layer "F.Cu") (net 6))
 (segment (start 160.4 62.57) (end 164.729 62.57) (width 0.2) (layer "F.Cu") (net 6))
 (segment (start 164.16 101.34) (end 146.56 101.34) (width 0.2) (layer "F.Cu") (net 6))
 (segment (start 144.924 92.611) (end 146.225 91.31) (width 0.2) (layer "F.Cu") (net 6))
 (segment (start 143.6745 62.83) (end 143.515 62.83) (width 0.2) (layer "F.Cu") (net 6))
 (segment (start 164.729 100.771) (end 164.16 101.34) (width 0.2) (layer "F.Cu") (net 6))
 (segment (start 160.38 62.59) (end 160.4 62.57) (width 0.2) (layer "F.Cu") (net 6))
 (segment (start 144.924 99.704) (end 144.924 92.611) (width 0.2) (layer "F.Cu") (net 6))
 (segment (start 145.93 62.83) (end 142.68 62.83) (width 0.2) (layer "F.Cu") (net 6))
 (segment (start 164.729 62.57) (end 164.729 100.771) (width 0.2) (layer "F.Cu") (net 6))
 (segment (start 143.7545 62.91) (end 143.6745 62.83) (width 0.2) (layer "F.Cu") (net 6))
 (segment (start 153.41 62.82) (end 145.94 62.82) (width 0.2) (layer "F.Cu") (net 6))
 (via (at 160.38 62.59) (size 0.6) (drill 0.3) (layers "F.Cu" "B.Cu") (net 6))
 (via (at 153.41 62.82) (size 0.6) (drill 0.3) (layers "F.Cu" "B.Cu") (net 6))
 (segment (start 160.38 62.59) (end 160.3 62.67) (width 0.2) (layer "B.Cu") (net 6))
 (segment (start 153.56 62.67) (end 153.41 62.82) (width 0.2) (layer "B.Cu") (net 6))
 (segment (start 160.3 62.67) (end 153.56 62.67) (width 0.2) (layer "B.Cu") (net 6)))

